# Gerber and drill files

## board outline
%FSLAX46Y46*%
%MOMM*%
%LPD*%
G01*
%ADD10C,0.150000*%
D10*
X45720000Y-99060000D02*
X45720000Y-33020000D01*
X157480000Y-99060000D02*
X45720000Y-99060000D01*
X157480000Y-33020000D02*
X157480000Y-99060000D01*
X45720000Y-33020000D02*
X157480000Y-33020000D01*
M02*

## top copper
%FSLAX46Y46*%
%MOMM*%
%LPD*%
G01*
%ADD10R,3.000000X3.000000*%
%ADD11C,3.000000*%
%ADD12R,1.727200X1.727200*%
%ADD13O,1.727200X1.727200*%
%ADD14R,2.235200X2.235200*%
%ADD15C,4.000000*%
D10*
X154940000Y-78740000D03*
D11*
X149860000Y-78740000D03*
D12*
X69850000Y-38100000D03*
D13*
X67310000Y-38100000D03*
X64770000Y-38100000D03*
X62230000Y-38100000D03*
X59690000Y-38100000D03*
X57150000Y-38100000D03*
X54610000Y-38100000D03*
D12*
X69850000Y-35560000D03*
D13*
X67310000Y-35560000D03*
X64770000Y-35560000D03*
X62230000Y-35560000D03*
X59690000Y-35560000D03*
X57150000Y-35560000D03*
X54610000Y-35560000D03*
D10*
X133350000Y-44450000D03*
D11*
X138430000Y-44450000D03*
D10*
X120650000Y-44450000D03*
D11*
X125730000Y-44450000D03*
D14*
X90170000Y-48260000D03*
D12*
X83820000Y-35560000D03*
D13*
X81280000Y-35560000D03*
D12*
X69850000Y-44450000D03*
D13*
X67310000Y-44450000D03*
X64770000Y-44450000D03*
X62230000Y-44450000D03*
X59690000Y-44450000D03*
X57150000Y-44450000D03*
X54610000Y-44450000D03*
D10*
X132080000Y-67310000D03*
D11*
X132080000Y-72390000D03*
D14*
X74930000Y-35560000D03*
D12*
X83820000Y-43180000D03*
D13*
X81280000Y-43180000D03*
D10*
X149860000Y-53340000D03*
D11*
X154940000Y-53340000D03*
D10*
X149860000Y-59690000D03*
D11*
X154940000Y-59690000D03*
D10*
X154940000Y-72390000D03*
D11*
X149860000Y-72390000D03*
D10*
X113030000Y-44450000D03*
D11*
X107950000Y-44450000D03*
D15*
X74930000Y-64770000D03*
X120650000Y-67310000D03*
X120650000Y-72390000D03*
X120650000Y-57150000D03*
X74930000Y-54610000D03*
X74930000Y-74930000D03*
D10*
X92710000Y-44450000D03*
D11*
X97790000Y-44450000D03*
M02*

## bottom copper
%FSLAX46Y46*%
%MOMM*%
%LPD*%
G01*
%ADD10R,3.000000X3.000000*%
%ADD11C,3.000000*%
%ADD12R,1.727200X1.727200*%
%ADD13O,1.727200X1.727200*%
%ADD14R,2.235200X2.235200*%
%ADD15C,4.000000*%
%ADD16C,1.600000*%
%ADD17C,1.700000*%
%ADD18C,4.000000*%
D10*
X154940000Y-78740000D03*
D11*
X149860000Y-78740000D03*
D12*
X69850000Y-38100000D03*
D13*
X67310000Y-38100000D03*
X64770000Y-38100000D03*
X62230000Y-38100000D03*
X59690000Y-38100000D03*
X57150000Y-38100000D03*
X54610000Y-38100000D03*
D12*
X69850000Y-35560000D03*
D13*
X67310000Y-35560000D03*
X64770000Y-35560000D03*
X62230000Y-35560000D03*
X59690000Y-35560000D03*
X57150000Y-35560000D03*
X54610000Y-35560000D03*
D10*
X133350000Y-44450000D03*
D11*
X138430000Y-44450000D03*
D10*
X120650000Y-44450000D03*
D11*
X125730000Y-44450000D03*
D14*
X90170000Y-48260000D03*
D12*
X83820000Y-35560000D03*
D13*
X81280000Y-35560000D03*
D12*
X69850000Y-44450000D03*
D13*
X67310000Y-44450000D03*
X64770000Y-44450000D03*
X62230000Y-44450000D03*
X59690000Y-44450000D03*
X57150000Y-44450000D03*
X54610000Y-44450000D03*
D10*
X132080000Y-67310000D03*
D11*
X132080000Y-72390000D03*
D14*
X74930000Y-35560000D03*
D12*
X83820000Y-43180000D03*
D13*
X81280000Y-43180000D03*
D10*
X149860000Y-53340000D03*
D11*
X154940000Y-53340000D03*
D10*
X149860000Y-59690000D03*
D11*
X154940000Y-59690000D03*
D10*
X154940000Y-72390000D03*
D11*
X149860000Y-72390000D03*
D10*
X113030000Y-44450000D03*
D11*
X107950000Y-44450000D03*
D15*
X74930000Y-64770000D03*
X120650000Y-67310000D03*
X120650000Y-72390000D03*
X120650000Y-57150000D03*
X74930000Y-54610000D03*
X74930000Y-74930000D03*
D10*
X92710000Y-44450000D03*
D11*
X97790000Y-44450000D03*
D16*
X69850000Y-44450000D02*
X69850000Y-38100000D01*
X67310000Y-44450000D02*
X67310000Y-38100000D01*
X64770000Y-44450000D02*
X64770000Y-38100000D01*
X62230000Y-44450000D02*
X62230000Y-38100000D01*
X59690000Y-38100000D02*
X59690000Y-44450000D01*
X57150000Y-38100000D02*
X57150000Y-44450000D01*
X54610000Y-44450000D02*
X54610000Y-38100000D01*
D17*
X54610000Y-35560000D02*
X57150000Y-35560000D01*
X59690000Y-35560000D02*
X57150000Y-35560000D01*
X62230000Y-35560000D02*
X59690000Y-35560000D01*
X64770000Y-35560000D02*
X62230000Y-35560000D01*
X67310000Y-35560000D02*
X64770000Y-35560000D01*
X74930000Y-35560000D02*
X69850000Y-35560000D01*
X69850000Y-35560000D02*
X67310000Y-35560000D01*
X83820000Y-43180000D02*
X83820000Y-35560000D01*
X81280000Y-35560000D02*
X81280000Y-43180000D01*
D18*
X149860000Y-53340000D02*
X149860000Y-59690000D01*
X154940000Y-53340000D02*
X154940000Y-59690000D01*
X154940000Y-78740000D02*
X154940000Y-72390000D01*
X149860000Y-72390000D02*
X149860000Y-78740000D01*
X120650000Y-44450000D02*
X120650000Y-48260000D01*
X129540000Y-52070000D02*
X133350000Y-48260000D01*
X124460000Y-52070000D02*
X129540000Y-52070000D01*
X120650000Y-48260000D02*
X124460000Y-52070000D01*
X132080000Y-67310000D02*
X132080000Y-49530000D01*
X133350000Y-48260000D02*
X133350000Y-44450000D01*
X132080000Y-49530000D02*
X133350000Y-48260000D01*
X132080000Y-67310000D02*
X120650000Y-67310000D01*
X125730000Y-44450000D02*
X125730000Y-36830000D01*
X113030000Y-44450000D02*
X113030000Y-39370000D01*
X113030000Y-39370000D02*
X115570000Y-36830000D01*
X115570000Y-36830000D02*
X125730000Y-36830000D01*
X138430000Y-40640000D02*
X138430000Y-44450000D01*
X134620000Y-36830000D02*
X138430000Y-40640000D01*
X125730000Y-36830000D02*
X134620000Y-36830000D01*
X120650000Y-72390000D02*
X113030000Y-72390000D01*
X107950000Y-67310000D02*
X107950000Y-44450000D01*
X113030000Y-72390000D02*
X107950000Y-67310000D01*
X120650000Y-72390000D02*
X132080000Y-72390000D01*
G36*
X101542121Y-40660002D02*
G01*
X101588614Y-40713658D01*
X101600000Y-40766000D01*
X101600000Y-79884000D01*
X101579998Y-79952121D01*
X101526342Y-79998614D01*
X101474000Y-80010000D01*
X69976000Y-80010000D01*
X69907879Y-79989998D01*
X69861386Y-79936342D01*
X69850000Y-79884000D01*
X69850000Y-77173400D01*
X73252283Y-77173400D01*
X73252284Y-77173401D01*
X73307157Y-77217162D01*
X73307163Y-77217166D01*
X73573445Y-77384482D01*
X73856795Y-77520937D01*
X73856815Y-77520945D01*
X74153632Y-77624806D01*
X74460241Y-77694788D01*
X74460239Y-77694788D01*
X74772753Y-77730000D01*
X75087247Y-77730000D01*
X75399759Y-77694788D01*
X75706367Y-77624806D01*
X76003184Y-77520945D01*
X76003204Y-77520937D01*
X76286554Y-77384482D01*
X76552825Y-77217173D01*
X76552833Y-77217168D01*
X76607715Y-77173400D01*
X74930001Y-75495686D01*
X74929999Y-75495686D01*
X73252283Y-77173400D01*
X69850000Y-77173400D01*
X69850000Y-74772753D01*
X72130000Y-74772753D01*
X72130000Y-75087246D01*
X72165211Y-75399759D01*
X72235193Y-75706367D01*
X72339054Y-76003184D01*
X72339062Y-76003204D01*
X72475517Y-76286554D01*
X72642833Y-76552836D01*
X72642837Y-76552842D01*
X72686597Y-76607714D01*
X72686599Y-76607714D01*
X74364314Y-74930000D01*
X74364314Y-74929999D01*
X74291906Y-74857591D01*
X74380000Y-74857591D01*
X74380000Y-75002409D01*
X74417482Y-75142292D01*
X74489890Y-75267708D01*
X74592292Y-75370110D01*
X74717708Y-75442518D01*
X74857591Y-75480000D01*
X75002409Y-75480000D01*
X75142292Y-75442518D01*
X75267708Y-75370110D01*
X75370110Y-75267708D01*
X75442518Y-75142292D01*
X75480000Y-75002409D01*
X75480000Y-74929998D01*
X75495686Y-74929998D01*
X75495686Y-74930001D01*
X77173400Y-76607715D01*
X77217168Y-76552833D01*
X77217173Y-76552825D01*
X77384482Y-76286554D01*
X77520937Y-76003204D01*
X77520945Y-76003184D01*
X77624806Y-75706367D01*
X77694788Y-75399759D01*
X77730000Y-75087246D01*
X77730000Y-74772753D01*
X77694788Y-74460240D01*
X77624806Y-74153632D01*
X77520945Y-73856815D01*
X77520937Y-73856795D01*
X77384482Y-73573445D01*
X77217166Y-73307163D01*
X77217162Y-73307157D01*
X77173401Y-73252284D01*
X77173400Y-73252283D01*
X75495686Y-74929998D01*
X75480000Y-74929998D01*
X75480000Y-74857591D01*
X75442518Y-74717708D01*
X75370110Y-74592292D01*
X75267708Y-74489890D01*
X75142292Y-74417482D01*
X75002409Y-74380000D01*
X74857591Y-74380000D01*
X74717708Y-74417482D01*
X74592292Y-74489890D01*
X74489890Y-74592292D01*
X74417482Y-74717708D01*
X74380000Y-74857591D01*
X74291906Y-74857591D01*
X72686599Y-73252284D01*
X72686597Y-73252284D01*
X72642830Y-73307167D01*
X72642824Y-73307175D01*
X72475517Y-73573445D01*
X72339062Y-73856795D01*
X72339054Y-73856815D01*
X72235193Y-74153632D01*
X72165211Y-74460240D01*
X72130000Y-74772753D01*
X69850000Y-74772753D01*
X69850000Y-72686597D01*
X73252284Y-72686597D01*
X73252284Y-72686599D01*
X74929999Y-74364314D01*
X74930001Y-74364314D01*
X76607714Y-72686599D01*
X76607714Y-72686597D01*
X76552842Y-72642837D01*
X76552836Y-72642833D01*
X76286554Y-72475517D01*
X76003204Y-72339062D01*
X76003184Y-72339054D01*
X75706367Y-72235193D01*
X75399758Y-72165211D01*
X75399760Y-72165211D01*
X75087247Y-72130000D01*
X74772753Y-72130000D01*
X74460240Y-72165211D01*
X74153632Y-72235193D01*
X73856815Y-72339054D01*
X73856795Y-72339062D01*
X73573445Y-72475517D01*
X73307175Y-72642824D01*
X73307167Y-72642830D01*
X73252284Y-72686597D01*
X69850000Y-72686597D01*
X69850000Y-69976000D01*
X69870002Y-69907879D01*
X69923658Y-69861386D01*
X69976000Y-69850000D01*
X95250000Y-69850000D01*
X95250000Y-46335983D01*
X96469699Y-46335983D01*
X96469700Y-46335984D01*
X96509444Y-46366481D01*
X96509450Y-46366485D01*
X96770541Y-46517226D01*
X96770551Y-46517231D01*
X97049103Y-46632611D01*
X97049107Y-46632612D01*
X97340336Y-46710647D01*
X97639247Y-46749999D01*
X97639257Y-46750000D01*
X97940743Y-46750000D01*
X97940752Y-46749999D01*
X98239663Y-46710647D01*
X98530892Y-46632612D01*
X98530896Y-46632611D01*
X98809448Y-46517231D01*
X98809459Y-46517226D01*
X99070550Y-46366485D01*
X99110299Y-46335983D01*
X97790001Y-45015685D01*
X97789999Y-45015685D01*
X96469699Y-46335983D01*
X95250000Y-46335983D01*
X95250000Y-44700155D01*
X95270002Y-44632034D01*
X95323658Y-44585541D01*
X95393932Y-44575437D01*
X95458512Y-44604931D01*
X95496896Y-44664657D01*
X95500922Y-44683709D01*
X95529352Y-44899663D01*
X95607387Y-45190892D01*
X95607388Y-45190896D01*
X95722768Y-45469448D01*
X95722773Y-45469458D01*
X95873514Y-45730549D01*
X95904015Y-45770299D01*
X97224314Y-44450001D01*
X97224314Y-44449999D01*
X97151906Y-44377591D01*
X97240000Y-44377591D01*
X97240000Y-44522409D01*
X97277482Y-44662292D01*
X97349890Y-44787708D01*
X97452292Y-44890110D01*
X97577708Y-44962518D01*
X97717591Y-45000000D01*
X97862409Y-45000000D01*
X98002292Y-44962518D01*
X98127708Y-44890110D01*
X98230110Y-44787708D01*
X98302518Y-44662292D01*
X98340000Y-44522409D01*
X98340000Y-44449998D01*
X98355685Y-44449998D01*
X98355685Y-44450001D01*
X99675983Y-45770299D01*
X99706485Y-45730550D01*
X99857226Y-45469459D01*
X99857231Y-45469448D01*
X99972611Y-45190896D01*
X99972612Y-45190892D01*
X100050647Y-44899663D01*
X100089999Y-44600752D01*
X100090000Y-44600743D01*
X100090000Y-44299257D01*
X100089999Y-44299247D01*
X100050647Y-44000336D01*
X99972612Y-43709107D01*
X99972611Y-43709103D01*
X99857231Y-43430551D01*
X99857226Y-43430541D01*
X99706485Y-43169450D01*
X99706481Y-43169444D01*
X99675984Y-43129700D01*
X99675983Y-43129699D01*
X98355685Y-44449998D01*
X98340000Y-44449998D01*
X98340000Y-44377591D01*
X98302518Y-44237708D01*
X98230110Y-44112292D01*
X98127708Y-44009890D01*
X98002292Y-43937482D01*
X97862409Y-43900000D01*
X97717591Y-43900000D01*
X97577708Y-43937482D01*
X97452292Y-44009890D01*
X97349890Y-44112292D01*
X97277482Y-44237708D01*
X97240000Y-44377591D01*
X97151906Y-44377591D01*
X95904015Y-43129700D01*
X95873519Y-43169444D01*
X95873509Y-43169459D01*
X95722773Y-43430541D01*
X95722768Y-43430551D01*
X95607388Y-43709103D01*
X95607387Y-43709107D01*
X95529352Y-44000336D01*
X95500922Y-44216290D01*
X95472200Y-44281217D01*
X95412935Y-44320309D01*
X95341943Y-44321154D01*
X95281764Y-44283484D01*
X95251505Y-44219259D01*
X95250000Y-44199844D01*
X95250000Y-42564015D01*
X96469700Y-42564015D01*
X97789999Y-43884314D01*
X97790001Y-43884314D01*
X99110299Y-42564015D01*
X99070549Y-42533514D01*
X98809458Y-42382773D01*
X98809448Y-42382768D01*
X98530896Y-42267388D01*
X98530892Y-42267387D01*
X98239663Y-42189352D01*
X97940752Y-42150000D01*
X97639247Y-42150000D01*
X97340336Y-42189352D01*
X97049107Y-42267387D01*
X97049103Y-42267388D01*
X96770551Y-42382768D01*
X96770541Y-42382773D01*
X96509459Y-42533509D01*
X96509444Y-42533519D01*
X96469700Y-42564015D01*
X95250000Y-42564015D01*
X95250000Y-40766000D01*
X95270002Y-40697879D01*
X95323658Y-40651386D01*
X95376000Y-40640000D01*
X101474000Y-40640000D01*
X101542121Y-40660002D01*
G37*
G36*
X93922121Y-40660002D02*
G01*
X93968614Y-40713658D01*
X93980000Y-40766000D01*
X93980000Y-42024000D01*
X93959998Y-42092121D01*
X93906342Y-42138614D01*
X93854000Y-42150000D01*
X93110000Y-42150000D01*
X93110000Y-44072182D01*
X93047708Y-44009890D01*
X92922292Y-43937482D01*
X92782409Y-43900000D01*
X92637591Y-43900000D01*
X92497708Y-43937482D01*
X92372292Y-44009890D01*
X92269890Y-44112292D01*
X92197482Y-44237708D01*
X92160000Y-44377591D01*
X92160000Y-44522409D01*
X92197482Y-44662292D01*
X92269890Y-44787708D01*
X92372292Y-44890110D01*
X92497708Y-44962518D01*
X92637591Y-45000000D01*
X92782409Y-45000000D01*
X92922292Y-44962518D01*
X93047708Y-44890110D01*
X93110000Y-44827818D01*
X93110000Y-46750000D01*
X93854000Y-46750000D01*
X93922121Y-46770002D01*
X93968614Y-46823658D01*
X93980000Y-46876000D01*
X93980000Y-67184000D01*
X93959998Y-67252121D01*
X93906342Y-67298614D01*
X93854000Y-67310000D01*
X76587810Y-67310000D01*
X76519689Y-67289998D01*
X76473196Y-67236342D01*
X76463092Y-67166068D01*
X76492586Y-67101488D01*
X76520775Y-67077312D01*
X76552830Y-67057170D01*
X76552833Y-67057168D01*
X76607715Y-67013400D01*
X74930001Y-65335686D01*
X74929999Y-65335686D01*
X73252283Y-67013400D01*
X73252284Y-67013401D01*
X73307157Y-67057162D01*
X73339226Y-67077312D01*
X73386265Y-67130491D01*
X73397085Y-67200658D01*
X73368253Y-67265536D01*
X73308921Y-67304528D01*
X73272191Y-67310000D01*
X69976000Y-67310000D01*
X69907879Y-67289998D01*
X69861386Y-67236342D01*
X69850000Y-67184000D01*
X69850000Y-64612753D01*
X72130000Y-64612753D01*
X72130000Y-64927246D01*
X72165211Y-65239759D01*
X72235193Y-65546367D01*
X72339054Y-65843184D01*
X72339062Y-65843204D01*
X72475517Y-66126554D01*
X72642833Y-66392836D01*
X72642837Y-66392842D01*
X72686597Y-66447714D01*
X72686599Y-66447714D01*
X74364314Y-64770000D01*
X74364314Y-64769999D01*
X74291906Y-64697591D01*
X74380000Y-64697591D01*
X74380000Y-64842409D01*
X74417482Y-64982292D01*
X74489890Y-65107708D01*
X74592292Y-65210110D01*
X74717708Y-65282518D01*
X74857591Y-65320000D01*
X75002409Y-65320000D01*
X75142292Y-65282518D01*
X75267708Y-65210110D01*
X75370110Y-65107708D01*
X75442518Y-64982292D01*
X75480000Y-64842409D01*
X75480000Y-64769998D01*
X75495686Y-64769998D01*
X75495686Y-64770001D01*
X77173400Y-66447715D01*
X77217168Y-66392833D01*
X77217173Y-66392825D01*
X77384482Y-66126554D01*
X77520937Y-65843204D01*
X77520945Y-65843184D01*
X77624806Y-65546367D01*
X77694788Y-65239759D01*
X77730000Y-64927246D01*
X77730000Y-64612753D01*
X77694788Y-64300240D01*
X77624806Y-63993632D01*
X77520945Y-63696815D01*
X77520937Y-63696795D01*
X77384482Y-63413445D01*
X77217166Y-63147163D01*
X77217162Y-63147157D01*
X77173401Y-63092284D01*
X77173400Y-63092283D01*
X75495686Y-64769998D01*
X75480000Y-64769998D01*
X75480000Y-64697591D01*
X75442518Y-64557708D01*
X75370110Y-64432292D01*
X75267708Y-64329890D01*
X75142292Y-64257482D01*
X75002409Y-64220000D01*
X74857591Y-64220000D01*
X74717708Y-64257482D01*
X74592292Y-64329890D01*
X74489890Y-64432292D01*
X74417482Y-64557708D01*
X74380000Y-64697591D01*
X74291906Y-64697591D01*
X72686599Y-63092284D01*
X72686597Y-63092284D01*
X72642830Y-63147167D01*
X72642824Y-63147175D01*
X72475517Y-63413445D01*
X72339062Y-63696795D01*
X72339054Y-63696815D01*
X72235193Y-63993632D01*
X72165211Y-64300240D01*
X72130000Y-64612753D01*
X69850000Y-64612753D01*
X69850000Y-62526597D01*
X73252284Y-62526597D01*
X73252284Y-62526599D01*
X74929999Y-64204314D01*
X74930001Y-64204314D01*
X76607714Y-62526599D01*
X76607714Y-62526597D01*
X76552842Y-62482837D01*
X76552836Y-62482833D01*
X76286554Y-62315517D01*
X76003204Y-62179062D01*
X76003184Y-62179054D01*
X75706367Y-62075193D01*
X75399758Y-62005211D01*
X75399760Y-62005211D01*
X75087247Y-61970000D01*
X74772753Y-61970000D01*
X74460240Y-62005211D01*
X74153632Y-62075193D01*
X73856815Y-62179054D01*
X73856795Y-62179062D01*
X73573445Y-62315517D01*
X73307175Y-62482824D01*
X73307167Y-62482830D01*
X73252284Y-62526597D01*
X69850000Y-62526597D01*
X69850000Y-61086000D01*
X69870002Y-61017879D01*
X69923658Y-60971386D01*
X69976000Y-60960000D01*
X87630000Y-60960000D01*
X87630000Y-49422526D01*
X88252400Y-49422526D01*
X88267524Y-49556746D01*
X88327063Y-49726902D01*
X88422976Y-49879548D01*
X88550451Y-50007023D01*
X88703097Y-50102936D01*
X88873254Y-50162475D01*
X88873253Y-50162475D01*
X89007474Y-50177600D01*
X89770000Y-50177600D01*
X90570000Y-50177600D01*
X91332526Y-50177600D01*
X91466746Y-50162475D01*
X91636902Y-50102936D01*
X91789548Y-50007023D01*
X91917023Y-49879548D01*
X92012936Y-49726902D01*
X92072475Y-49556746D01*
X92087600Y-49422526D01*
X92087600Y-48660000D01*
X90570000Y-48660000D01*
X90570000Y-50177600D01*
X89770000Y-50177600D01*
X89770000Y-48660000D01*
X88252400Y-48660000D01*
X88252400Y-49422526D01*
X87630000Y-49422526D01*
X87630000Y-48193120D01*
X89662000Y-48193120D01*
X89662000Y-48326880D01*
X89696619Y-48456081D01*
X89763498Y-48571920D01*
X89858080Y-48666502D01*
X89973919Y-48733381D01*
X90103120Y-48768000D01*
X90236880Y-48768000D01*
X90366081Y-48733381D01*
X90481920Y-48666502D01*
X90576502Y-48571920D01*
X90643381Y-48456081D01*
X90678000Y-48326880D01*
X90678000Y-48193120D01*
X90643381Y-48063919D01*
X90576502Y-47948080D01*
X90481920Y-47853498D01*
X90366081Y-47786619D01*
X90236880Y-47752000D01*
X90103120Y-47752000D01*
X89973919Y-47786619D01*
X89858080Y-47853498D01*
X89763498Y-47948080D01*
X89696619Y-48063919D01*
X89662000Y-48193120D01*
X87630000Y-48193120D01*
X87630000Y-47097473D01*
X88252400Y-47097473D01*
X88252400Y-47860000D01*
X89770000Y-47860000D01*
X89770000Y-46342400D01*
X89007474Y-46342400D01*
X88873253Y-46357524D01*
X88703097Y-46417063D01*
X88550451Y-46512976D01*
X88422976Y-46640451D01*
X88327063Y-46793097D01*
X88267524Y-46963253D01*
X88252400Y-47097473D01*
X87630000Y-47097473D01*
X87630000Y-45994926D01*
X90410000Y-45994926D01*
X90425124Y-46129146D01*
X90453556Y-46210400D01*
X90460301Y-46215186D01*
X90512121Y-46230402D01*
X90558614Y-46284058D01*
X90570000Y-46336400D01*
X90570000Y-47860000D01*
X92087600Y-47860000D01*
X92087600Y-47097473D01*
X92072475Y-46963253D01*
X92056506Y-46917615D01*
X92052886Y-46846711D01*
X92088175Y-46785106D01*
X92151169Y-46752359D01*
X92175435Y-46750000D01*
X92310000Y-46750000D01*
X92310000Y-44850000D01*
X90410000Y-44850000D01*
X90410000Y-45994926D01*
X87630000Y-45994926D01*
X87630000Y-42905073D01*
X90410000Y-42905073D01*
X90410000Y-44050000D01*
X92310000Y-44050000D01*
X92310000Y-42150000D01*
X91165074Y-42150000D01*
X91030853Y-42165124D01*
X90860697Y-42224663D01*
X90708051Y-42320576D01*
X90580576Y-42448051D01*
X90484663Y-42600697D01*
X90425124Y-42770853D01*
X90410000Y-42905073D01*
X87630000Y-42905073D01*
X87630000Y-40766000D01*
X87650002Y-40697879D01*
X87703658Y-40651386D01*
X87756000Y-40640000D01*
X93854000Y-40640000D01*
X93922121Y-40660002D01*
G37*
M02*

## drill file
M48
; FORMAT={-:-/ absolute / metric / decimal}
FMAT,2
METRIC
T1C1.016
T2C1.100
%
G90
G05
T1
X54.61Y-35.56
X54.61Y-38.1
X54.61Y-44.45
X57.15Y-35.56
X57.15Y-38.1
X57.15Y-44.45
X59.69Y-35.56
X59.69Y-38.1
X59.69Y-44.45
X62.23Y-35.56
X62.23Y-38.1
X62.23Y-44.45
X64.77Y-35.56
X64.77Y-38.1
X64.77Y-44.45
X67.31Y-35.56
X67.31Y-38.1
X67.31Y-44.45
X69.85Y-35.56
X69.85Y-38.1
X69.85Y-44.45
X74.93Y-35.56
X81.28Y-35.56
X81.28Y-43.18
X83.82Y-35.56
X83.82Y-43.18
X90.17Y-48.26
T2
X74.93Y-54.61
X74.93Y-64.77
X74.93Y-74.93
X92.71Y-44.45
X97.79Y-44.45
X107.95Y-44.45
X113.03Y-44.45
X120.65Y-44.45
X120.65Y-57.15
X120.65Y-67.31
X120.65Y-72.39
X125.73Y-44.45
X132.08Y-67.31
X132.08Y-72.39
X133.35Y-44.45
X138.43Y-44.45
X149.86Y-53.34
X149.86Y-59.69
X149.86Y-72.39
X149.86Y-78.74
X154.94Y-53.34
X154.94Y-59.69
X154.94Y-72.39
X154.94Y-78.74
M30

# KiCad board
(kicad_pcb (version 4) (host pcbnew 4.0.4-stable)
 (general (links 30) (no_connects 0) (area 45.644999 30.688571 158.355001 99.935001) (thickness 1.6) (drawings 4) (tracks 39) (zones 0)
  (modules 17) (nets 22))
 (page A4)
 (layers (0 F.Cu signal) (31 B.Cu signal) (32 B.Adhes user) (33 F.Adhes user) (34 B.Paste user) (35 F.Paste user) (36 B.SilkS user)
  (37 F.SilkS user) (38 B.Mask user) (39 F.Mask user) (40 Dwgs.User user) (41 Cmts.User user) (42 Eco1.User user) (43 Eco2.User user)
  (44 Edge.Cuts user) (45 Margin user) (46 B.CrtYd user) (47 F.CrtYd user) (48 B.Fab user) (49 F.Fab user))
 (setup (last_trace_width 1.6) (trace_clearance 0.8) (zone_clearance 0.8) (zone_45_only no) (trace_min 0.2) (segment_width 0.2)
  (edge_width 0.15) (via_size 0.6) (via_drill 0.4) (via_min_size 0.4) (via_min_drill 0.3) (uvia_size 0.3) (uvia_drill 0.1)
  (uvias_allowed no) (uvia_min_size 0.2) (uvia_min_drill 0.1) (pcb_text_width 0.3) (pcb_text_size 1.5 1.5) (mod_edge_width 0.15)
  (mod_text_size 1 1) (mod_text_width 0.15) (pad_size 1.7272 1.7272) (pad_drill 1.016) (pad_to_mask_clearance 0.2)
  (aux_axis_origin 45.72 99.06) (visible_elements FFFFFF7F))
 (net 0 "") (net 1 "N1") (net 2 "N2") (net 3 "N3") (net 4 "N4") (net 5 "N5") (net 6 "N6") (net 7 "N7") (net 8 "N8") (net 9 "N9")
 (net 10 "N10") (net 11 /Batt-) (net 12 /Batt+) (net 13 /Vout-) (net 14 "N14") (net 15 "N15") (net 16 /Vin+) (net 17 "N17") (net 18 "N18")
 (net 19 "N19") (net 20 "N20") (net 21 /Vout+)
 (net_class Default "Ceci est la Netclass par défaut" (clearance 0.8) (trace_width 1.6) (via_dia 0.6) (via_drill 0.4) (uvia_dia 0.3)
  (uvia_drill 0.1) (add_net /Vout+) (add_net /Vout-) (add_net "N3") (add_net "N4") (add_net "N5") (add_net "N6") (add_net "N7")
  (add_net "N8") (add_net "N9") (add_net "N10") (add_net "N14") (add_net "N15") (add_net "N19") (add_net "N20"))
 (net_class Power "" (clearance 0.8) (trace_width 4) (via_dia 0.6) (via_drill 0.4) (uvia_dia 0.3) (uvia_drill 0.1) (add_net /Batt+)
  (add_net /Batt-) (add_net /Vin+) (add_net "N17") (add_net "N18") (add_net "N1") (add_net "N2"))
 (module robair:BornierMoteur (layer F.Cu) (at 152.4 78.74 180)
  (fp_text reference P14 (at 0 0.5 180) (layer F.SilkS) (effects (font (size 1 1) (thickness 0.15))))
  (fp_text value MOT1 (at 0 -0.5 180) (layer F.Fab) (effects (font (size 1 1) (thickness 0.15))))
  (pad 1 thru_hole rect (at -2.54 0 180) (size 3 3) (drill 1.1) (layers *.Cu *.Mask) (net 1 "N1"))
  (pad 2 thru_hole circle (at 2.54 0 180) (size 3 3) (drill 1.1) (layers *.Cu *.Mask) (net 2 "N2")))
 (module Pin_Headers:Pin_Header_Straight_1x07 (layer F.Cu) (at 69.85 38.1 270)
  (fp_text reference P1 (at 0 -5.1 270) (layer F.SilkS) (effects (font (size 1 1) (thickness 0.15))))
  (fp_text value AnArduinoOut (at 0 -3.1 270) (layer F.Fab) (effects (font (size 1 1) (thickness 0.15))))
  (pad 1 thru_hole rect (at 0 0 270) (size 1.7272 1.7272) (drill 1.016) (layers *.Cu *.Mask F.SilkS) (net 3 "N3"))
  (pad 2 thru_hole oval (at 0 2.54 270) (size 1.7272 1.7272) (drill 1.016) (layers *.Cu *.Mask F.SilkS) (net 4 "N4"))
  (pad 3 thru_hole oval (at 0 5.08 270) (size 1.7272 1.7272) (drill 1.016) (layers *.Cu *.Mask F.SilkS) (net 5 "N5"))
  (pad 4 thru_hole oval (at 0 7.62 270) (size 1.7272 1.7272) (drill 1.016) (layers *.Cu *.Mask F.SilkS) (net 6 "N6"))
  (pad 5 thru_hole oval (at 0 10.16 270) (size 1.7272 1.7272) (drill 1.016) (layers *.Cu *.Mask F.SilkS) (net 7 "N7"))
  (pad 6 thru_hole oval (at 0 12.7 270) (size 1.7272 1.7272) (drill 1.016) (layers *.Cu *.Mask F.SilkS) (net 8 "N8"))
  (pad 7 thru_hole oval (at 0 15.24 270) (size 1.7272 1.7272) (drill 1.016) (layers *.Cu *.Mask F.SilkS) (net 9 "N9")))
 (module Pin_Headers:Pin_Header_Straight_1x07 (layer F.Cu) (at 69.85 35.56 270)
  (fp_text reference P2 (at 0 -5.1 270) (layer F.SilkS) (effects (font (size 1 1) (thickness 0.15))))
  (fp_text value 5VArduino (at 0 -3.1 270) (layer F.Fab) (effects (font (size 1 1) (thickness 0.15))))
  (pad 1 thru_hole rect (at 0 0 270) (size 1.7272 1.7272) (drill 1.016) (layers *.Cu *.Mask F.SilkS) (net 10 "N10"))
  (pad 2 thru_hole oval (at 0 2.54 270) (size 1.7272 1.7272) (drill 1.016) (layers *.Cu *.Mask F.SilkS) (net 10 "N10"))
  (pad 3 thru_hole oval (at 0 5.08 270) (size 1.7272 1.7272) (drill 1.016) (layers *.Cu *.Mask F.SilkS) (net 10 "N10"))
  (pad 4 thru_hole oval (at 0 7.62 270) (size 1.7272 1.7272) (drill 1.016) (layers *.Cu *.Mask F.SilkS) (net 10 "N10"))
  (pad 5 thru_hole oval (at 0 10.16 270) (size 1.7272 1.7272) (drill 1.016) (layers *.Cu *.Mask F.SilkS) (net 10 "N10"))
  (pad 6 thru_hole oval (at 0 12.7 270) (size 1.7272 1.7272) (drill 1.016) (layers *.Cu *.Mask F.SilkS) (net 10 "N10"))
  (pad 7 thru_hole oval (at 0 15.24 270) (size 1.7272 1.7272) (drill 1.016) (layers *.Cu *.Mask F.SilkS) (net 10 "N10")))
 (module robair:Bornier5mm (layer F.Cu) (at 135.89 44.45)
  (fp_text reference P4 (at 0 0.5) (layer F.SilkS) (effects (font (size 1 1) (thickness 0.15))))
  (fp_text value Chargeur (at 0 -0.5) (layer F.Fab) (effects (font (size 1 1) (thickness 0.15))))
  (pad 1 thru_hole rect (at -2.54 0) (size 3 3) (drill 1.1) (layers *.Cu *.Mask) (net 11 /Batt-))
  (pad 2 thru_hole circle (at 2.54 0) (size 3 3) (drill 1.1) (layers *.Cu *.Mask) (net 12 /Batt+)))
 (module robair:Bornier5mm (layer F.Cu) (at 123.19 44.45)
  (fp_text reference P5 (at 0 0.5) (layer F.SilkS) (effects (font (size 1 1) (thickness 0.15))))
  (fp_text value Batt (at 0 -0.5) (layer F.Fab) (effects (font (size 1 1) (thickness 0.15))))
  (pad 1 thru_hole rect (at -2.54 0) (size 3 3) (drill 1.1) (layers *.Cu *.Mask) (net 11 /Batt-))
  (pad 2 thru_hole circle (at 2.54 0) (size 3 3) (drill 1.1) (layers *.Cu *.Mask) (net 12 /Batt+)))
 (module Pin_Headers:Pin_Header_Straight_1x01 (layer F.Cu) (at 90.17 48.26)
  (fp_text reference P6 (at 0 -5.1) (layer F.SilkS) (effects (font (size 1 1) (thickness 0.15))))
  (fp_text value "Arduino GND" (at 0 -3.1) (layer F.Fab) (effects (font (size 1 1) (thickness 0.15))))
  (pad 1 thru_hole rect (at 0 0) (size 2.2352 2.2352) (drill 1.016) (layers *.Cu *.Mask F.SilkS) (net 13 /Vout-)))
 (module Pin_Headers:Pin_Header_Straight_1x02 (layer F.Cu) (at 83.82 35.56 270)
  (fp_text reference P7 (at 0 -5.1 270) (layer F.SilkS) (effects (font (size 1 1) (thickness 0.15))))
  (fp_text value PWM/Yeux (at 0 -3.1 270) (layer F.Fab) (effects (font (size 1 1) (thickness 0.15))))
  (pad 1 thru_hole rect (at 0 0 270) (size 1.7272 1.7272) (drill 1.016) (layers *.Cu *.Mask F.SilkS) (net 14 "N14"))
  (pad 2 thru_hole oval (at 0 2.54 270) (size 1.7272 1.7272) (drill 1.016) (layers *.Cu *.Mask F.SilkS) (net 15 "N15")))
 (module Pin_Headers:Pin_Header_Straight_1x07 (layer F.Cu) (at 69.85 44.45 270)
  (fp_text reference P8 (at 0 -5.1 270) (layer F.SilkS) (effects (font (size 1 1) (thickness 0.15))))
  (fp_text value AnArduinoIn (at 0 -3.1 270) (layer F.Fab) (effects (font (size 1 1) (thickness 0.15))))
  (pad 1 thru_hole rect (at 0 0 270) (size 1.7272 1.7272) (drill 1.016) (layers *.Cu *.Mask F.SilkS) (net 3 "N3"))
  (pad 2 thru_hole oval (at 0 2.54 270) (size 1.7272 1.7272) (drill 1.016) (layers *.Cu *.Mask F.SilkS) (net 4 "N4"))
  (pad 3 thru_hole oval (at 0 5.08 270) (size 1.7272 1.7272) (drill 1.016) (layers *.Cu *.Mask F.SilkS) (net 5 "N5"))
  (pad 4 thru_hole oval (at 0 7.62 270) (size 1.7272 1.7272) (drill 1.016) (layers *.Cu *.Mask F.SilkS) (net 6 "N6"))
  (pad 5 thru_hole oval (at 0 10.16 270) (size 1.7272 1.7272) (drill 1.016) (layers *.Cu *.Mask F.SilkS) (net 7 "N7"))
  (pad 6 thru_hole oval (at 0 12.7 270) (size 1.7272 1.7272) (drill 1.016) (layers *.Cu *.Mask F.SilkS) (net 8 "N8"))
  (pad 7 thru_hole oval (at 0 15.24 270) (size 1.7272 1.7272) (drill 1.016) (layers *.Cu *.Mask F.SilkS) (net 9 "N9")))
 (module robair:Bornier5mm (layer F.Cu) (at 132.08 69.85 270)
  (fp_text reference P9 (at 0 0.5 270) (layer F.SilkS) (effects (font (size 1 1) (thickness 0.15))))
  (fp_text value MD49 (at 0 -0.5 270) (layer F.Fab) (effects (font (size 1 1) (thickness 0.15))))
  (pad 1 thru_hole rect (at -2.54 0 270) (size 3 3) (drill 1.1) (layers *.Cu *.Mask) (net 11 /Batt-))
  (pad 2 thru_hole circle (at 2.54 0 270) (size 3 3) (drill 1.1) (layers *.Cu *.Mask) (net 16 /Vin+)))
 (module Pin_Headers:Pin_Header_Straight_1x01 (layer F.Cu) (at 74.93 35.56 270)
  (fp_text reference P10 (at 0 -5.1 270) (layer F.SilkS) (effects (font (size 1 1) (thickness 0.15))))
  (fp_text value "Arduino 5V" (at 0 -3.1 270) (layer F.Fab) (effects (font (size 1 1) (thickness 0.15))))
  (pad 1 thru_hole rect (at 0 0 270) (size 2.2352 2.2352) (drill 1.016) (layers *.Cu *.Mask F.SilkS) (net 10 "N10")))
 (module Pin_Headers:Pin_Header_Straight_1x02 (layer F.Cu) (at 83.82 43.18 270)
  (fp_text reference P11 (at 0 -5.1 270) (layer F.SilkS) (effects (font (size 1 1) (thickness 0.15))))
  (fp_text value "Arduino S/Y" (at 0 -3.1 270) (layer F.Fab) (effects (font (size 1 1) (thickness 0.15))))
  (pad 1 thru_hole rect (at 0 0 270) (size 1.7272 1.7272) (drill 1.016) (layers *.Cu *.Mask F.SilkS) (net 14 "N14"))
  (pad 2 thru_hole oval (at 0 2.54 270) (size 1.7272 1.7272) (drill 1.016) (layers *.Cu *.Mask F.SilkS) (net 15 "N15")))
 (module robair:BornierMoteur (layer F.Cu) (at 152.4 53.34)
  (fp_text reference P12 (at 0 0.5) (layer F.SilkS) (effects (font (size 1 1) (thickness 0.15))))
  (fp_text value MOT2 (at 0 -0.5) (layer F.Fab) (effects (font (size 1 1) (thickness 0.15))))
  (pad 1 thru_hole rect (at -2.54 0) (size 3 3) (drill 1.1) (layers *.Cu *.Mask) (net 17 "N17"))
  (pad 2 thru_hole circle (at 2.54 0) (size 3 3) (drill 1.1) (layers *.Cu *.Mask) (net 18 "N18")))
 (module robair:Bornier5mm (layer F.Cu) (at 152.4 59.69)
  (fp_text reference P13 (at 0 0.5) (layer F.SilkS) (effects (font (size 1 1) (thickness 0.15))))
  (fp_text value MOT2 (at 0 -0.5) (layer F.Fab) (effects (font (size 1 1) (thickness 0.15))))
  (pad 1 thru_hole rect (at -2.54 0) (size 3 3) (drill 1.1) (layers *.Cu *.Mask) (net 17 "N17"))
  (pad 2 thru_hole circle (at 2.54 0) (size 3 3) (drill 1.1) (layers *.Cu *.Mask) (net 18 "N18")))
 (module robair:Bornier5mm (layer F.Cu) (at 152.4 72.39 180)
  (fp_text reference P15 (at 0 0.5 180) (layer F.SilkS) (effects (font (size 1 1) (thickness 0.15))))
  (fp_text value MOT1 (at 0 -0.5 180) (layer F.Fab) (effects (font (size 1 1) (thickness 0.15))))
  (pad 1 thru_hole rect (at -2.54 0 180) (size 3 3) (drill 1.1) (layers *.Cu *.Mask) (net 1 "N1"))
  (pad 2 thru_hole circle (at 2.54 0 180) (size 3 3) (drill 1.1) (layers *.Cu *.Mask) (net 2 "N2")))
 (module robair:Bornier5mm (layer B.Cu) (at 110.49 44.45 180)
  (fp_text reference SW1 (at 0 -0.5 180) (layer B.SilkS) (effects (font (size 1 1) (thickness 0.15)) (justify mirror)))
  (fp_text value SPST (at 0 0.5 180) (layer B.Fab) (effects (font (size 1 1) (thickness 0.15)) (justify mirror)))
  (pad 1 thru_hole rect (at -2.54 0 180) (size 3 3) (drill 1.1) (layers *.Cu *.Mask) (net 12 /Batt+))
  (pad 2 thru_hole circle (at 2.54 0 180) (size 3 3) (drill 1.1) (layers *.Cu *.Mask) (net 16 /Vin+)))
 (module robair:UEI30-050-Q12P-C (layer F.Cu) (at 97.79 64.77)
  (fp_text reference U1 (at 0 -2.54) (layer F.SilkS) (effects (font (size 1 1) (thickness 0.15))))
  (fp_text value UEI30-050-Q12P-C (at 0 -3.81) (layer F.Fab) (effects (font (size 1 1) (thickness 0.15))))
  (pad 5 thru_hole circle (at -22.86 0) (size 4 4) (drill 1.1) (layers *.Cu *.Mask) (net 13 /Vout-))
  (pad 2 thru_hole circle (at 22.86 2.54) (size 4 4) (drill 1.1) (layers *.Cu *.Mask) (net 11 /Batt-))
  (pad 1 thru_hole circle (at 22.86 7.62) (size 4 4) (drill 1.1) (layers *.Cu *.Mask) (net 16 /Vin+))
  (pad 3 thru_hole circle (at 22.86 -7.62) (size 4 4) (drill 1.1) (layers *.Cu *.Mask) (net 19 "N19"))
  (pad 6 thru_hole circle (at -22.86 -10.16) (size 4 4) (drill 1.1) (layers *.Cu *.Mask) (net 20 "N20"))
  (pad 4 thru_hole circle (at -22.86 10.16) (size 4 4) (drill 1.1) (layers *.Cu *.Mask) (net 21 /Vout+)))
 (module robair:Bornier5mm (layer F.Cu) (at 95.25 44.45)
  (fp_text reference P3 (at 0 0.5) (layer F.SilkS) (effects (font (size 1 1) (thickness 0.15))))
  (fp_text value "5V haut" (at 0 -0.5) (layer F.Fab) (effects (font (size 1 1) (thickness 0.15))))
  (pad 1 thru_hole rect (at -2.54 0) (size 3 3) (drill 1.1) (layers *.Cu *.Mask) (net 13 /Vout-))
  (pad 2 thru_hole circle (at 2.54 0) (size 3 3) (drill 1.1) (layers *.Cu *.Mask) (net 21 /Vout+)))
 (gr_line (start 45.72 99.06) (end 45.72 33.02) (angle 90) (layer Edge.Cuts) (width 0.15))
 (gr_line (start 157.48 99.06) (end 45.72 99.06) (angle 90) (layer Edge.Cuts) (width 0.15))
 (gr_line (start 157.48 33.02) (end 157.48 99.06) (angle 90) (layer Edge.Cuts) (width 0.15))
 (gr_line (start 45.72 33.02) (end 157.48 33.02) (angle 90) (layer Edge.Cuts) (width 0.15))
 (segment (start 69.85 44.45) (end 69.85 38.1) (width 1.6) (layer B.Cu) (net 3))
 (segment (start 67.31 44.45) (end 67.31 38.1) (width 1.6) (layer B.Cu) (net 4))
 (segment (start 64.77 44.45) (end 64.77 38.1) (width 1.6) (layer B.Cu) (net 5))
 (segment (start 62.23 44.45) (end 62.23 38.1) (width 1.6) (layer B.Cu) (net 6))
 (segment (start 59.69 38.1) (end 59.69 44.45) (width 1.6) (layer B.Cu) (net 7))
 (segment (start 57.15 38.1) (end 57.15 44.45) (width 1.6) (layer B.Cu) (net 8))
 (segment (start 54.61 44.45) (end 54.61 38.1) (width 1.6) (layer B.Cu) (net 9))
 (segment (start 54.61 35.56) (end 57.15 35.56) (width 1.7) (layer B.Cu) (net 10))
 (segment (start 59.69 35.56) (end 57.15 35.56) (width 1.7) (layer B.Cu) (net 10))
 (segment (start 62.23 35.56) (end 59.69 35.56) (width 1.7) (layer B.Cu) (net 10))
 (segment (start 64.77 35.56) (end 62.23 35.56) (width 1.7) (layer B.Cu) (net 10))
 (segment (start 67.31 35.56) (end 64.77 35.56) (width 1.7) (layer B.Cu) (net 10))
 (segment (start 74.93 35.56) (end 69.85 35.56) (width 1.7) (layer B.Cu) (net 10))
 (segment (start 69.85 35.56) (end 67.31 35.56) (width 1.7) (layer B.Cu) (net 10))
 (segment (start 83.82 43.18) (end 83.82 35.56) (width 1.7) (layer B.Cu) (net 14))
 (segment (start 81.28 35.56) (end 81.28 43.18) (width 1.7) (layer B.Cu) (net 15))
 (segment (start 149.86 53.34) (end 149.86 59.69) (width 4) (layer B.Cu) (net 17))
 (segment (start 154.94 53.34) (end 154.94 59.69) (width 4) (layer B.Cu) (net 18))
 (segment (start 154.94 78.74) (end 154.94 72.39) (width 4) (layer B.Cu) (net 1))
 (segment (start 149.86 72.39) (end 149.86 78.74) (width 4) (layer B.Cu) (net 2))
 (segment (start 120.65 44.45) (end 120.65 48.26) (width 4) (layer B.Cu) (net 11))
 (segment (start 129.54 52.07) (end 133.35 48.26) (width 4) (layer B.Cu) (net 11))
 (segment (start 124.46 52.07) (end 129.54 52.07) (width 4) (layer B.Cu) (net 11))
 (segment (start 120.65 48.26) (end 124.46 52.07) (width 4) (layer B.Cu) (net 11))
 (segment (start 132.08 67.31) (end 132.08 49.53) (width 4) (layer B.Cu) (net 11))
 (segment (start 133.35 48.26) (end 133.35 44.45) (width 4) (layer B.Cu) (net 11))
 (segment (start 132.08 49.53) (end 133.35 48.26) (width 4) (layer B.Cu) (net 11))
 (segment (start 132.08 67.31) (end 120.65 67.31) (width 4) (layer B.Cu) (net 11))
 (segment (start 125.73 44.45) (end 125.73 36.83) (width 4) (layer B.Cu) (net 12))
 (segment (start 113.03 44.45) (end 113.03 39.37) (width 4) (layer B.Cu) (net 12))
 (segment (start 113.03 39.37) (end 115.57 36.83) (width 4) (layer B.Cu) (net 12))
 (segment (start 115.57 36.83) (end 125.73 36.83) (width 4) (layer B.Cu) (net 12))
 (segment (start 138.43 40.64) (end 138.43 44.45) (width 4) (layer B.Cu) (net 12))
 (segment (start 134.62 36.83) (end 138.43 40.64) (width 4) (layer B.Cu) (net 12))
 (segment (start 125.73 36.83) (end 134.62 36.83) (width 4) (layer B.Cu) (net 12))
 (segment (start 120.65 72.39) (end 113.03 72.39) (width 4) (layer B.Cu) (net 16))
 (segment (start 107.95 67.31) (end 107.95 44.45) (width 4) (layer B.Cu) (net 16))
 (segment (start 113.03 72.39) (end 107.95 67.31) (width 4) (layer B.Cu) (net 16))
 (segment (start 120.65 72.39) (end 132.08 72.39) (width 4) (layer B.Cu) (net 16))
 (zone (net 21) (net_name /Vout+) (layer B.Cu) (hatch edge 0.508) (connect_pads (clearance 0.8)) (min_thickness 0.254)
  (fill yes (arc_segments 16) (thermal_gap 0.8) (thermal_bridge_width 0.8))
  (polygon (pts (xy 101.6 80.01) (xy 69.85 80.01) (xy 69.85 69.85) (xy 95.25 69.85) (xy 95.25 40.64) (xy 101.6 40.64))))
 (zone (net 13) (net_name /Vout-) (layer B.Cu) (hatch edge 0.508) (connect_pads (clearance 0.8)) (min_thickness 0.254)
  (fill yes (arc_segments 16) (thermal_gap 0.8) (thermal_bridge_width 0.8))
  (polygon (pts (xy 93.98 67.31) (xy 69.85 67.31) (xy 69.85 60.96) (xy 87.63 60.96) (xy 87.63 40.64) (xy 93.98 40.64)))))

